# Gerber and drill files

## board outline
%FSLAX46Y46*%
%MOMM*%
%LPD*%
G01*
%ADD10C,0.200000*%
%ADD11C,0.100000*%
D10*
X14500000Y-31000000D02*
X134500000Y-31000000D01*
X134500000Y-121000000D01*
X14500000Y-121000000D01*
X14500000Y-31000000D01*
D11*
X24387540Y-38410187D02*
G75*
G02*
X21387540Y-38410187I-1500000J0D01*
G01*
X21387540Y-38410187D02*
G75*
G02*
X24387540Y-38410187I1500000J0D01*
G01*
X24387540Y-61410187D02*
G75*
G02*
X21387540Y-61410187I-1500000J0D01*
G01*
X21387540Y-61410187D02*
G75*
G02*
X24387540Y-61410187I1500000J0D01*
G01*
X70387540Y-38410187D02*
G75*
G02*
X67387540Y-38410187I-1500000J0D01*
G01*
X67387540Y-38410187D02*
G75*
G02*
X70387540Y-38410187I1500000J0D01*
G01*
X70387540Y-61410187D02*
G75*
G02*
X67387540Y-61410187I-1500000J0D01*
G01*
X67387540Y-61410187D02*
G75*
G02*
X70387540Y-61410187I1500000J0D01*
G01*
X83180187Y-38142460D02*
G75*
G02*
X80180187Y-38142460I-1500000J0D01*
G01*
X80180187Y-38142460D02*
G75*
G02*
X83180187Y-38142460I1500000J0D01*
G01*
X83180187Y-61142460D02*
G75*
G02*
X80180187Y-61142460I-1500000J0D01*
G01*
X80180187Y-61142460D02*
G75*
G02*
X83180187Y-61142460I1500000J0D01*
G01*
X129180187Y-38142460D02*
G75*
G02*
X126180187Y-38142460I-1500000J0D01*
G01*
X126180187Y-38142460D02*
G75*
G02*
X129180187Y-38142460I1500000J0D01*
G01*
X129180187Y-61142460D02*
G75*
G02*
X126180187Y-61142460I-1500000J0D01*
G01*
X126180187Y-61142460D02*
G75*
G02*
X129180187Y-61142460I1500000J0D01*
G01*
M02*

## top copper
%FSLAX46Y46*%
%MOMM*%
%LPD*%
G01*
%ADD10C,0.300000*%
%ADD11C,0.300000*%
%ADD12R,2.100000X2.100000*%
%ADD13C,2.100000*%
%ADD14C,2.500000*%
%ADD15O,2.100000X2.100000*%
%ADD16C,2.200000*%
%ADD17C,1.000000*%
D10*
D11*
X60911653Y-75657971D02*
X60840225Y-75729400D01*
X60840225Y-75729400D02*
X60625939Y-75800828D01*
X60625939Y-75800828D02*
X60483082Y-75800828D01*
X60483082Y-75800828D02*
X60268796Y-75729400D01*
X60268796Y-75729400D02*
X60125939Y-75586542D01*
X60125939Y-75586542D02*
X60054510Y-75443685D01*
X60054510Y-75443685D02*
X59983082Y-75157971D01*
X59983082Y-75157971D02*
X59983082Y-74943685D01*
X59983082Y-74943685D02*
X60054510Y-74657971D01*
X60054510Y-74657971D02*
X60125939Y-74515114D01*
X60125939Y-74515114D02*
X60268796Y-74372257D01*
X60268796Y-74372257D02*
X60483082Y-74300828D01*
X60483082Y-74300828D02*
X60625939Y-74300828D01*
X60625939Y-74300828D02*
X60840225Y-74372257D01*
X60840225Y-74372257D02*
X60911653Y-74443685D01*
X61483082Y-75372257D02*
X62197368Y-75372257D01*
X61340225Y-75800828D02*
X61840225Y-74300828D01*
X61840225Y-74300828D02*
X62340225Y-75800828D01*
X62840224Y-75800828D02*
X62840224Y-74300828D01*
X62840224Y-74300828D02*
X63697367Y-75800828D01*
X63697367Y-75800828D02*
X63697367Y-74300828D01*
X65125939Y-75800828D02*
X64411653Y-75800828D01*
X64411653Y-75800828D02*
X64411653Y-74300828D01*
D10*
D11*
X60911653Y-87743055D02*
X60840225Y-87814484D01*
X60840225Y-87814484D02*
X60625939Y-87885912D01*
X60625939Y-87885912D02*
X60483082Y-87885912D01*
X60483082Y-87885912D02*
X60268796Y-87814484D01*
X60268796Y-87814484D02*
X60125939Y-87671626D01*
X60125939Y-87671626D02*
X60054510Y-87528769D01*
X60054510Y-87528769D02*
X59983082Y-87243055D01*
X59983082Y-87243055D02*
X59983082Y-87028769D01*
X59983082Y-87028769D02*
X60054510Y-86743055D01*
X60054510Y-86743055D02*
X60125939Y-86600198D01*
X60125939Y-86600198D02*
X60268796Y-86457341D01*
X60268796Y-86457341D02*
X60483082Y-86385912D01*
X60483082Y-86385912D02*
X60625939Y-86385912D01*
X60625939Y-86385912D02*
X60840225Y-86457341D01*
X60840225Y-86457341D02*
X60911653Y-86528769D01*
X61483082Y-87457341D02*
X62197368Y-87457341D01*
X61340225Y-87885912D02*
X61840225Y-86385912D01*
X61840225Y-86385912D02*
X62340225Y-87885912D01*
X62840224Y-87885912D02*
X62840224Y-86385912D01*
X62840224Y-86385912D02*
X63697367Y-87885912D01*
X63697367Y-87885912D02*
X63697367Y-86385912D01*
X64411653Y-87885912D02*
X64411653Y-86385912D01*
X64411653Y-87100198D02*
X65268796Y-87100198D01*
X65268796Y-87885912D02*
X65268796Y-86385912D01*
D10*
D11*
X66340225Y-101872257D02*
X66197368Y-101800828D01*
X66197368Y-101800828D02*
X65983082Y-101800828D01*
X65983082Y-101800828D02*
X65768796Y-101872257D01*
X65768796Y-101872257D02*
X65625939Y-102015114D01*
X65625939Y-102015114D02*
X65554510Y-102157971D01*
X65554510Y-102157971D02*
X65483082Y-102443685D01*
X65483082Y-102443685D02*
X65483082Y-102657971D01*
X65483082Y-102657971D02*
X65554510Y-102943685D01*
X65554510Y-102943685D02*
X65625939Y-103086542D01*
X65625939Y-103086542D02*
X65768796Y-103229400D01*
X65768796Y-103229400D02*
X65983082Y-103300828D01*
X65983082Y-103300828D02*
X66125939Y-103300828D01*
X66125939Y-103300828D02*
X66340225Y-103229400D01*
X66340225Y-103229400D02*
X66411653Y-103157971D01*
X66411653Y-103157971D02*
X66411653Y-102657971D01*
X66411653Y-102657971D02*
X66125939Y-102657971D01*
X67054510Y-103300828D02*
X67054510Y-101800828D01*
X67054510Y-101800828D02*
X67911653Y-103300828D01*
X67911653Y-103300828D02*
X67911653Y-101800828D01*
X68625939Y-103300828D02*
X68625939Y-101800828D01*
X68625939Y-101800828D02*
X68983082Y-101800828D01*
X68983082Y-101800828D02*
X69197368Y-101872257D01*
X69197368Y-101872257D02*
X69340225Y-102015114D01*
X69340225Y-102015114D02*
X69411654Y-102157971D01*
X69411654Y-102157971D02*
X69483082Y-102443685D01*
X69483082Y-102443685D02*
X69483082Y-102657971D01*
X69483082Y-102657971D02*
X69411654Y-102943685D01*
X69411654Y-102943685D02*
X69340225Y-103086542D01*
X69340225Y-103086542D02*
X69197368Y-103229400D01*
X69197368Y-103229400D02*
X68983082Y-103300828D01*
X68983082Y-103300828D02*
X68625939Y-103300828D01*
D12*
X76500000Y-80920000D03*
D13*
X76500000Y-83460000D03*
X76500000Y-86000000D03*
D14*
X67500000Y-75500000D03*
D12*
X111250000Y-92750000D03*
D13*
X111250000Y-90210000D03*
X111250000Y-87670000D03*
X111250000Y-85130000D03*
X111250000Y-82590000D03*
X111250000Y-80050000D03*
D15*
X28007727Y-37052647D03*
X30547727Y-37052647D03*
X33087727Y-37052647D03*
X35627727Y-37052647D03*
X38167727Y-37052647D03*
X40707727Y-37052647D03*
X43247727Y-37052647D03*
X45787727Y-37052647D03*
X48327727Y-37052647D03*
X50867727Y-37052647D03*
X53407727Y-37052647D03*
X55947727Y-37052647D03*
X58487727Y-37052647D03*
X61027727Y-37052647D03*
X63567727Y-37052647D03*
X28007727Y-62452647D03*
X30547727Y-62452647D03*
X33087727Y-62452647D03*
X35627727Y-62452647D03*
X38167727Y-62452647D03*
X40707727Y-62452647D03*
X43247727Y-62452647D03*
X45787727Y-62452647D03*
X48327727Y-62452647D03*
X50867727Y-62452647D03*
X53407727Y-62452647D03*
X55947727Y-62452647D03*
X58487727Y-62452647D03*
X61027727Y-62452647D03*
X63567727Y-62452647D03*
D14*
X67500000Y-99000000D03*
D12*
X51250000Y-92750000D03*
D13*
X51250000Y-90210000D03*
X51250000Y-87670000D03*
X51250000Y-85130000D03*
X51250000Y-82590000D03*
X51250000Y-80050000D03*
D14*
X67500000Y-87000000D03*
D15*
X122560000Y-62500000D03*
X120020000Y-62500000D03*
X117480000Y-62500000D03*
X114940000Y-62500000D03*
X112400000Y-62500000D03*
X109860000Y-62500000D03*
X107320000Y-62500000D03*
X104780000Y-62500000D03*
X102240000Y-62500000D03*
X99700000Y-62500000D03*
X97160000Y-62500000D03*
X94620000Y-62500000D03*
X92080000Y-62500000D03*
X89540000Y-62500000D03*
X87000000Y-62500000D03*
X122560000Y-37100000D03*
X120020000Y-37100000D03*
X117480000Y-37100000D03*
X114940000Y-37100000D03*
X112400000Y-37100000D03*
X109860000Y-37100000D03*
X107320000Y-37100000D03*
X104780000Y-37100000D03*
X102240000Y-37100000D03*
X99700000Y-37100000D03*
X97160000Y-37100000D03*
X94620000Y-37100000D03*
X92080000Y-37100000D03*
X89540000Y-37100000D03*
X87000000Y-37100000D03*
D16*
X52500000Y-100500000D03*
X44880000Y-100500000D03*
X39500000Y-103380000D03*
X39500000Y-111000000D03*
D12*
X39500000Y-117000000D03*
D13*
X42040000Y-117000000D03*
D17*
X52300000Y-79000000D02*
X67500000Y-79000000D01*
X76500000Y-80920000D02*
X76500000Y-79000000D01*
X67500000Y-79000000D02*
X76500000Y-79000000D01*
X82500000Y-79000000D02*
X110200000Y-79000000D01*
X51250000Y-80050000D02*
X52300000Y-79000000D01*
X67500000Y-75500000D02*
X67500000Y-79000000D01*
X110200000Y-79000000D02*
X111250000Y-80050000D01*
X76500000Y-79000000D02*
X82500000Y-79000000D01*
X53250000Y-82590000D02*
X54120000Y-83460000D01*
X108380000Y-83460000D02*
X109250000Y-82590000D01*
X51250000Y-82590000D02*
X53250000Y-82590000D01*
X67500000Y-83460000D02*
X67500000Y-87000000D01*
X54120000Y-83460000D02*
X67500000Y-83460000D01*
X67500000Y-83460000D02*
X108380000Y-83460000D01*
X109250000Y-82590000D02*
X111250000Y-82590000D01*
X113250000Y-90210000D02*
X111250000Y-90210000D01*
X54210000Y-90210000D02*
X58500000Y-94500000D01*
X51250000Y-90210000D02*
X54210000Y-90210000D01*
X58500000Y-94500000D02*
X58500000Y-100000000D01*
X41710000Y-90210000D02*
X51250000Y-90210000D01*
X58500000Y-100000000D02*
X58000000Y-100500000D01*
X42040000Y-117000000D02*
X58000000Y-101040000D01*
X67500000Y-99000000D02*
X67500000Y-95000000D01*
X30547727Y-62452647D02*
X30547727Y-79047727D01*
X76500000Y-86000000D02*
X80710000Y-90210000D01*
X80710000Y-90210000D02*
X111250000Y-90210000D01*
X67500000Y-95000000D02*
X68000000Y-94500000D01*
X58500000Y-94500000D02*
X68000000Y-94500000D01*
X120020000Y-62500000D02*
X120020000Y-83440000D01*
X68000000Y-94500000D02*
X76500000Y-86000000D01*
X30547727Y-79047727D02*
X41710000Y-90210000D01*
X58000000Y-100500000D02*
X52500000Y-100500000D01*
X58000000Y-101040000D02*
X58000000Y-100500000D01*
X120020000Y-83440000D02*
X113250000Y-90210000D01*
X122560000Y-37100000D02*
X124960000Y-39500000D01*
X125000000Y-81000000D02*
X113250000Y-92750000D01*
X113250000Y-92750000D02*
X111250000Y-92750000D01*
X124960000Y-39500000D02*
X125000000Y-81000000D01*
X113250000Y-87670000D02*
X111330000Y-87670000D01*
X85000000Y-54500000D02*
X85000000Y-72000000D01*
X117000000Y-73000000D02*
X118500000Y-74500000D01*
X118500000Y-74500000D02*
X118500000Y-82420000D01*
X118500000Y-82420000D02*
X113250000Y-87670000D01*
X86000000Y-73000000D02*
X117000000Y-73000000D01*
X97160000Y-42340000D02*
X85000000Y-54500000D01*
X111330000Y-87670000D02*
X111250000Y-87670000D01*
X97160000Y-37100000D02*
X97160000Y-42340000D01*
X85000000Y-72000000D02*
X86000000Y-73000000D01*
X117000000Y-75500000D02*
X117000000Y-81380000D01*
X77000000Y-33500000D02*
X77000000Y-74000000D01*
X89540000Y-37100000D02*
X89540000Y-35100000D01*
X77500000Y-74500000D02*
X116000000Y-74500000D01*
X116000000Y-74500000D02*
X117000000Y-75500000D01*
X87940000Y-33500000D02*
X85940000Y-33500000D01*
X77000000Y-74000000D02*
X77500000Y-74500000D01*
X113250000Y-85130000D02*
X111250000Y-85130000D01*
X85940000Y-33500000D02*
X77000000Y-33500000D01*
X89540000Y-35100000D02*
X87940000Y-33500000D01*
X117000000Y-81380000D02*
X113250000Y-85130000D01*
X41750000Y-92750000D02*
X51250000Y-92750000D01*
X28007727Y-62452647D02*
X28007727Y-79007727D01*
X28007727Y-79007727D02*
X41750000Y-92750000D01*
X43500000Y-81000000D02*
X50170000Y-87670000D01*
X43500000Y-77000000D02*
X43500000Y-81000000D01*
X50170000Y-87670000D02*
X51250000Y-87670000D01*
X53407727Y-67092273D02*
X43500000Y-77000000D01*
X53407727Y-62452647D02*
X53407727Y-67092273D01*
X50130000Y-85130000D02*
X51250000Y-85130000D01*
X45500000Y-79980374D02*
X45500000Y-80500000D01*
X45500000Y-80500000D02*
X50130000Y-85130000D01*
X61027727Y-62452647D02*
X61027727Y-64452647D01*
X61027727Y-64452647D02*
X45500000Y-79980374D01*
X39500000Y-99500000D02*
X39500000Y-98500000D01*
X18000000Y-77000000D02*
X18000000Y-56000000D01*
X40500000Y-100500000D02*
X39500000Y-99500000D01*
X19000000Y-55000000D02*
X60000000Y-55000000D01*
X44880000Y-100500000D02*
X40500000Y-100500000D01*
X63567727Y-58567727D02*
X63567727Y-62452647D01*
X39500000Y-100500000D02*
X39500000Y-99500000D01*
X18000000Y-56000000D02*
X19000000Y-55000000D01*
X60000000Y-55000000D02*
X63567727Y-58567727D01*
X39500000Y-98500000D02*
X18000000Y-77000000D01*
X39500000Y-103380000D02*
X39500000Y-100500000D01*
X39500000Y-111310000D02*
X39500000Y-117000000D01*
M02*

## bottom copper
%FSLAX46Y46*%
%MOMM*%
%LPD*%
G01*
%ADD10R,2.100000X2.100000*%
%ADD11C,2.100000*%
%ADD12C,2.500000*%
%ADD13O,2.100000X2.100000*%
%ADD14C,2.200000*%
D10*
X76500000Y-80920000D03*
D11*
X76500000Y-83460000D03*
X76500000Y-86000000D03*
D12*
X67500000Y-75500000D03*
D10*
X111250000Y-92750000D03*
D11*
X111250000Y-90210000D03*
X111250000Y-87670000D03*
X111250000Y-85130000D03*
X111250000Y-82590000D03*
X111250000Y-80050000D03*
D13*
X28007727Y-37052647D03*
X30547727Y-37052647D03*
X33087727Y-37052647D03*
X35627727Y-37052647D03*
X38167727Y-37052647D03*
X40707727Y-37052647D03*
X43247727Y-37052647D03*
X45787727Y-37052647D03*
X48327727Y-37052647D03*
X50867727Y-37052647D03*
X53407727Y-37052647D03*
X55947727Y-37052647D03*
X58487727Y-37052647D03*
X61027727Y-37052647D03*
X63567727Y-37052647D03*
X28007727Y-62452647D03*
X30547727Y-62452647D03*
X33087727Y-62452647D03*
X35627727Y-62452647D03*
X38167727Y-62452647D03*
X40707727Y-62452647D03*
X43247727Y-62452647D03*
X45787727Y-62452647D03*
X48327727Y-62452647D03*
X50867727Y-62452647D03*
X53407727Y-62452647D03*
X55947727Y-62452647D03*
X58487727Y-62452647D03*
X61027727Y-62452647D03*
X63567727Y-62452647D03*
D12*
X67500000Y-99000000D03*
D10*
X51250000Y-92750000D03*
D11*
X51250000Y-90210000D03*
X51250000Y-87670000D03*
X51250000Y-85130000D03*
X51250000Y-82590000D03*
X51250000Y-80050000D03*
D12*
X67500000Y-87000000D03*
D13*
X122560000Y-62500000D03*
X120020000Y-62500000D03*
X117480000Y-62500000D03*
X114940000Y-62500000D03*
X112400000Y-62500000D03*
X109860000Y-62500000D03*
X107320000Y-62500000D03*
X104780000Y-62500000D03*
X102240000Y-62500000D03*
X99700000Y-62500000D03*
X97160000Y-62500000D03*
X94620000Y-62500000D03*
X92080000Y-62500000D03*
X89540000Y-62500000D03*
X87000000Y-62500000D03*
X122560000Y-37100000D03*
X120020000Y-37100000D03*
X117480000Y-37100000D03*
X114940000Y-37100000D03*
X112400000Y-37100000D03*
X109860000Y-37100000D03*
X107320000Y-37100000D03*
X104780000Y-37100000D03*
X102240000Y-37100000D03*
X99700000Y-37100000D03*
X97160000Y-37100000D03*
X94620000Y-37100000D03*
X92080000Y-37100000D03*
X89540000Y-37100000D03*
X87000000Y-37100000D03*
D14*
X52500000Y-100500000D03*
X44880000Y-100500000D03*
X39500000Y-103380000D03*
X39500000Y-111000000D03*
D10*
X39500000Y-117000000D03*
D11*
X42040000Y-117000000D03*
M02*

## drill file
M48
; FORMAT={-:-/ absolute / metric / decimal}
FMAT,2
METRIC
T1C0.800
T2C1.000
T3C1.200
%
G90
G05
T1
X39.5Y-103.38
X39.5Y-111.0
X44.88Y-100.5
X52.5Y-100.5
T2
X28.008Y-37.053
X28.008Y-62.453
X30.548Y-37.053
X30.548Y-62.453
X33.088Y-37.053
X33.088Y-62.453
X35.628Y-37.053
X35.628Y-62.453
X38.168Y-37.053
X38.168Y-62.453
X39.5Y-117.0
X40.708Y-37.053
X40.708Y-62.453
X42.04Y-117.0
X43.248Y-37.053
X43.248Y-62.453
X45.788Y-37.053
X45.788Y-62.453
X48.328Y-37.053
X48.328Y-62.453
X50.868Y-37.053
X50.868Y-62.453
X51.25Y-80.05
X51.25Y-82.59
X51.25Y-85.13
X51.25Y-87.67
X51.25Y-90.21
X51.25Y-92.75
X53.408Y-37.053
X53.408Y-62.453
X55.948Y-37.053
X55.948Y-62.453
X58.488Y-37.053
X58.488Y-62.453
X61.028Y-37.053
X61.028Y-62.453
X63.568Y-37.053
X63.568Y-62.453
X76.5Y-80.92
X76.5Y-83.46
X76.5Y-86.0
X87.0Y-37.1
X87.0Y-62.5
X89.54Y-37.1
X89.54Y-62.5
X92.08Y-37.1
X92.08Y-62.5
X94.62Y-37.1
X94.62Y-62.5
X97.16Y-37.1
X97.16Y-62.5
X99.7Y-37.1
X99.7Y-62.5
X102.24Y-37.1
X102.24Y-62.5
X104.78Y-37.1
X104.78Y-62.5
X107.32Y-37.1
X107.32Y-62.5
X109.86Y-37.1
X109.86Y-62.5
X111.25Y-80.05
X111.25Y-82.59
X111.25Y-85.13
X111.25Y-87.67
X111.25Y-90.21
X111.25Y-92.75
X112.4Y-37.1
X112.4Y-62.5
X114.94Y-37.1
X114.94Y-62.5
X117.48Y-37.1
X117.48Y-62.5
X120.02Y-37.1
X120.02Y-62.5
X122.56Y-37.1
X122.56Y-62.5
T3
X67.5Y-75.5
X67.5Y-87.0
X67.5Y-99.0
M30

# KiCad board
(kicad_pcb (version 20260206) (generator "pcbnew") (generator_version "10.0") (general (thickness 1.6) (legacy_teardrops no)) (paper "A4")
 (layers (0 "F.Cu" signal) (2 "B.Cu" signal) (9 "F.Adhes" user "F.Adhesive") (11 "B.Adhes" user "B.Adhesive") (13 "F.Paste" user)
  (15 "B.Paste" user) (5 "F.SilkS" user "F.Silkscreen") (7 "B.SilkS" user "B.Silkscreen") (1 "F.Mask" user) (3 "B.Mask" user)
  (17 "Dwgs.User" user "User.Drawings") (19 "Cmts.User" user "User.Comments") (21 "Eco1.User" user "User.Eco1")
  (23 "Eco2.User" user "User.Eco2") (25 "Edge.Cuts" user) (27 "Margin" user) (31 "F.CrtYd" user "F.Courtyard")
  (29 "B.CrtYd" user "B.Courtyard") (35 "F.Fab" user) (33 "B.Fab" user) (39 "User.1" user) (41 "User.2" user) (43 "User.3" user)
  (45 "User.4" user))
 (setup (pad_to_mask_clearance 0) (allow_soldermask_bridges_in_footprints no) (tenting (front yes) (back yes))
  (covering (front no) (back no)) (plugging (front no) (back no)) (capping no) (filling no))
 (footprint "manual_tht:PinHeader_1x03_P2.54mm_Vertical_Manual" (layer "F.Cu") (at 76.5 80.92)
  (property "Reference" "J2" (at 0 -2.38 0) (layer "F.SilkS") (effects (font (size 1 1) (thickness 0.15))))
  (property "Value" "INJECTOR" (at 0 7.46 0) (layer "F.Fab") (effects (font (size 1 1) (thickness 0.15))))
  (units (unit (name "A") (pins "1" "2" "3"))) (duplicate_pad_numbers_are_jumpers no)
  (pad "1" thru_hole rect (at 0 0) (size 2.1 2.1) (drill 1) (layers "*.Cu" "*.Mask") (remove_unused_layers no) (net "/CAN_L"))
  (pad "2" thru_hole circle (at 0 2.54) (size 2.1 2.1) (drill 1) (layers "*.Cu" "*.Mask") (remove_unused_layers no) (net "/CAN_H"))
  (pad "3" thru_hole circle (at 0 5.08) (size 2.1 2.1) (drill 1) (layers "*.Cu" "*.Mask") (remove_unused_layers no) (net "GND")))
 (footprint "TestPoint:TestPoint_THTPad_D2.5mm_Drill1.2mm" (layer "F.Cu") (at 67.5 75.5)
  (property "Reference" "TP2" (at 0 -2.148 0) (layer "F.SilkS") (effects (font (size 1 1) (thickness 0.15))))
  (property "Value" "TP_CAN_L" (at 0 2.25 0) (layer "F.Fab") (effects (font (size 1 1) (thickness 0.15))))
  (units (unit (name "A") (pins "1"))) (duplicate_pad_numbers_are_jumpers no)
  (pad "1" thru_hole circle (at 0 0) (size 2.5 2.5) (drill 1.2) (layers "*.Cu" "*.Mask") (remove_unused_layers no) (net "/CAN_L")))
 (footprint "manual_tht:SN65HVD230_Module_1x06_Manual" (layer "F.Cu") (at 111.25 92.75 180)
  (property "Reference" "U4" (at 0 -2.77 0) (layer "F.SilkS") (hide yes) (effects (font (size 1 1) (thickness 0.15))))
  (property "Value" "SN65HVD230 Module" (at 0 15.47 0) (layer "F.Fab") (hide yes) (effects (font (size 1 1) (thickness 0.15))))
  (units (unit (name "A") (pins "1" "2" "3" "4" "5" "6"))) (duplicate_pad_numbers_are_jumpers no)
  (pad "1" thru_hole rect (at 0 0 180) (size 2.1 2.1) (drill 1) (layers "*.Cu" "*.Mask") (remove_unused_layers no) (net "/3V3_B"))
  (pad "2" thru_hole circle (at 0 2.54 180) (size 2.1 2.1) (drill 1) (layers "*.Cu" "*.Mask") (remove_unused_layers no) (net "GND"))
  (pad "3" thru_hole circle (at 0 5.08 180) (size 2.1 2.1) (drill 1) (layers "*.Cu" "*.Mask") (remove_unused_layers no) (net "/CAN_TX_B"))
  (pad "4" thru_hole circle (at 0 7.62 180) (size 2.1 2.1) (drill 1) (layers "*.Cu" "*.Mask") (remove_unused_layers no) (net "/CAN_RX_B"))
  (pad "5" thru_hole circle (at 0 10.16 180) (size 2.1 2.1) (drill 1) (layers "*.Cu" "*.Mask") (remove_unused_layers no) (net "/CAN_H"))
  (pad "6" thru_hole circle (at 0 12.7 180) (size 2.1 2.1) (drill 1) (layers "*.Cu" "*.Mask") (remove_unused_layers no) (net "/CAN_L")))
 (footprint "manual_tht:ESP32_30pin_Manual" (layer "F.Cu") (at 45.02754 48.980187 -90)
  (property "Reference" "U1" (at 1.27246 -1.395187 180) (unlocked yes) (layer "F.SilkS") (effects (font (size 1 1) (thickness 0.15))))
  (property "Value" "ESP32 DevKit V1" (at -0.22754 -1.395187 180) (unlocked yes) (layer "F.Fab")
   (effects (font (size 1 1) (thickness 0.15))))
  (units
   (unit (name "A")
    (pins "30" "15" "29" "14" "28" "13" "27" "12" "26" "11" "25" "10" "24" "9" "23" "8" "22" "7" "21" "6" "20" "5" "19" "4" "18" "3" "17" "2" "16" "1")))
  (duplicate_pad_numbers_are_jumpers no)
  (fp_circle (center -10.57 22.14) (end -10.57 23.64) (stroke (width 0.1) (type default)) (fill no) (layer "Edge.Cuts"))
  (fp_circle (center 12.43 22.14) (end 12.43 23.64) (stroke (width 0.1) (type default)) (fill no) (layer "Edge.Cuts"))
  (fp_circle (center -10.57 -23.86) (end -10.57 -22.36) (stroke (width 0.1) (type default)) (fill no) (layer "Edge.Cuts"))
  (fp_circle (center 12.43 -23.86) (end 12.43 -22.36) (stroke (width 0.1) (type default)) (fill no) (layer "Edge.Cuts"))
  (pad "1" thru_hole oval (at -11.92754 17.019813 180) (size 2.1 2.1) (drill 1) (layers "*.Cu" "*.Mask") (remove_unused_layers no)
   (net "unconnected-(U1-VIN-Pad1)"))
  (pad "2" thru_hole oval (at -11.92754 14.479813 180) (size 2.1 2.1) (drill 1) (layers "*.Cu" "*.Mask") (remove_unused_layers no)
   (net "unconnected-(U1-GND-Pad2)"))
  (pad "3" thru_hole oval (at -11.92754 11.939813 180) (size 2.1 2.1) (drill 1) (layers "*.Cu" "*.Mask") (remove_unused_layers no)
   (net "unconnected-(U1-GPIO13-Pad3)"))
  (pad "4" thru_hole oval (at -11.92754 9.399813 180) (size 2.1 2.1) (drill 1) (layers "*.Cu" "*.Mask") (remove_unused_layers no)
   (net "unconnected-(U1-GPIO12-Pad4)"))
  (pad "5" thru_hole oval (at -11.92754 6.859813 180) (size 2.1 2.1) (drill 1) (layers "*.Cu" "*.Mask") (remove_unused_layers no)
   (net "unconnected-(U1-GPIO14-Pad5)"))
  (pad "6" thru_hole oval (at -11.92754 4.319813 180) (size 2.1 2.1) (drill 1) (layers "*.Cu" "*.Mask") (remove_unused_layers no)
   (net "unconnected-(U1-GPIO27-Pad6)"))
  (pad "7" thru_hole oval (at -11.92754 1.779813 180) (size 2.1 2.1) (drill 1) (layers "*.Cu" "*.Mask") (remove_unused_layers no)
   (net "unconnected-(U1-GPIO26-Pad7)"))
  (pad "8" thru_hole oval (at -11.92754 -0.760187 180) (size 2.1 2.1) (drill 1) (layers "*.Cu" "*.Mask") (remove_unused_layers no)
   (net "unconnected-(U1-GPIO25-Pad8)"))
  (pad "9" thru_hole oval (at -11.92754 -3.300187 180) (size 2.1 2.1) (drill 1) (layers "*.Cu" "*.Mask") (remove_unused_layers no)
   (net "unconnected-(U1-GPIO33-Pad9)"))
  (pad "10" thru_hole oval (at -11.92754 -5.840187 180) (size 2.1 2.1) (drill 1) (layers "*.Cu" "*.Mask") (remove_unused_layers no)
   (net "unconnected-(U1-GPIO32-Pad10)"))
  (pad "11" thru_hole oval (at -11.92754 -8.380187 180) (size 2.1 2.1) (drill 1) (layers "*.Cu" "*.Mask") (remove_unused_layers no)
   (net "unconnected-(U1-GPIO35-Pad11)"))
  (pad "12" thru_hole oval (at -11.92754 -10.920187 180) (size 2.1 2.1) (drill 1) (layers "*.Cu" "*.Mask") (remove_unused_layers no)
   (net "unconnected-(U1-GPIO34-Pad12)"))
  (pad "13" thru_hole oval (at -11.92754 -13.460187 180) (size 2.1 2.1) (drill 1) (layers "*.Cu" "*.Mask") (remove_unused_layers no)
   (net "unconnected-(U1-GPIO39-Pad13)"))
  (pad "14" thru_hole oval (at -11.92754 -16.000187 180) (size 2.1 2.1) (drill 1) (layers "*.Cu" "*.Mask") (remove_unused_layers no)
   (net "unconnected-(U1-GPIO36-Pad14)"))
  (pad "15" thru_hole oval (at -11.92754 -18.540187 180) (size 2.1 2.1) (drill 1) (layers "*.Cu" "*.Mask") (remove_unused_layers no)
   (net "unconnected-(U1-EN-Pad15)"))
  (pad "16" thru_hole oval (at 13.47246 17.019813 180) (size 2.1 2.1) (drill 1) (layers "*.Cu" "*.Mask") (remove_unused_layers no)
   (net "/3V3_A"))
  (pad "17" thru_hole oval (at 13.47246 14.479813 180) (size 2.1 2.1) (drill 1) (layers "*.Cu" "*.Mask") (remove_unused_layers no)
   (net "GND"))
  (pad "18" thru_hole oval (at 13.47246 11.939813 180) (size 2.1 2.1) (drill 1) (layers "*.Cu" "*.Mask") (remove_unused_layers no)
   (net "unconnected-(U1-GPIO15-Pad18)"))
  (pad "19" thru_hole oval (at 13.47246 9.399813 180) (size 2.1 2.1) (drill 1) (layers "*.Cu" "*.Mask") (remove_unused_layers no)
   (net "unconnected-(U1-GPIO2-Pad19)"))
  (pad "20" thru_hole oval (at 13.47246 6.859813 180) (size 2.1 2.1) (drill 1) (layers "*.Cu" "*.Mask" "Dwgs.User")
   (remove_unused_layers no) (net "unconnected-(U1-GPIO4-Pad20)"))
  (pad "21" thru_hole oval (at 13.47246 4.319813 180) (size 2.1 2.1) (drill 1) (layers "*.Cu" "*.Mask") (remove_unused_layers no)
   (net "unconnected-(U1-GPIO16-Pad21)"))
  (pad "22" thru_hole oval (at 13.47246 1.779813 180) (size 2.1 2.1) (drill 1) (layers "*.Cu" "*.Mask") (remove_unused_layers no)
   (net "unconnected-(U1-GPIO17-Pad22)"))
  (pad "23" thru_hole oval (at 13.47246 -0.760187 180) (size 2.1 2.1) (drill 1) (layers "*.Cu" "*.Mask") (remove_unused_layers no)
   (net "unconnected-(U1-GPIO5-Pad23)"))
  (pad "24" thru_hole oval (at 13.47246 -3.300187 180) (size 2.1 2.1) (drill 1) (layers "*.Cu" "*.Mask") (remove_unused_layers no)
   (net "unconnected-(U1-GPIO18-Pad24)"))
  (pad "25" thru_hole oval (at 13.47246 -5.840187 180) (size 2.1 2.1) (drill 1) (layers "*.Cu" "*.Mask") (remove_unused_layers no)
   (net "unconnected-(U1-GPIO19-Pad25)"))
  (pad "26" thru_hole oval (at 13.47246 -8.380187 180) (size 2.1 2.1) (drill 1) (layers "*.Cu" "*.Mask") (remove_unused_layers no)
   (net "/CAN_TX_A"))
  (pad "27" thru_hole oval (at 13.47246 -10.920187 180) (size 2.1 2.1) (drill 1) (layers "*.Cu" "*.Mask") (remove_unused_layers no)
   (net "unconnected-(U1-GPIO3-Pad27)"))
  (pad "28" thru_hole oval (at 13.47246 -13.460187 180) (size 2.1 2.1) (drill 1) (layers "*.Cu" "*.Mask") (remove_unused_layers no)
   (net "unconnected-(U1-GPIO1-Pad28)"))
  (pad "29" thru_hole oval (at 13.47246 -16.000187 180) (size 2.1 2.1) (drill 1) (layers "*.Cu" "*.Mask") (remove_unused_layers no)
   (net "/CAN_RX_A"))
  (pad "30" thru_hole oval (at 13.47246 -18.540187 180) (size 2.1 2.1) (drill 1) (layers "*.Cu" "*.Mask") (remove_unused_layers no)
   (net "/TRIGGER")))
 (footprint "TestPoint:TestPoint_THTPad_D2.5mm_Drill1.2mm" (layer "F.Cu") (at 67.5 99)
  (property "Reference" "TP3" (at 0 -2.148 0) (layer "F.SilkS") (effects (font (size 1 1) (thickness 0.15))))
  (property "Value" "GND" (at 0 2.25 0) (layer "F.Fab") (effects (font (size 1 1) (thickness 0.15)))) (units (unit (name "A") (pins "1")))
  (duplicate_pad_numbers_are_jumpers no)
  (pad "1" thru_hole circle (at 0 0) (size 2.5 2.5) (drill 1.2) (layers "*.Cu" "*.Mask") (remove_unused_layers no) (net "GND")))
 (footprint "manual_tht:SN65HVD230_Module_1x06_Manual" (layer "F.Cu") (at 51.25 92.75 180)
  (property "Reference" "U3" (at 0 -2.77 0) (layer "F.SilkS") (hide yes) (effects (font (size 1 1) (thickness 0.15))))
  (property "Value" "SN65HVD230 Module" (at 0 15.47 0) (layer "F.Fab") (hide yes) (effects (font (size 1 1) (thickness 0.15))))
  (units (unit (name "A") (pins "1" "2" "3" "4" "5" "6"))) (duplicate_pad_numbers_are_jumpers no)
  (pad "1" thru_hole rect (at 0 0 180) (size 2.1 2.1) (drill 1) (layers "*.Cu" "*.Mask") (remove_unused_layers no) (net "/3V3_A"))
  (pad "2" thru_hole circle (at 0 2.54 180) (size 2.1 2.1) (drill 1) (layers "*.Cu" "*.Mask") (remove_unused_layers no) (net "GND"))
  (pad "3" thru_hole circle (at 0 5.08 180) (size 2.1 2.1) (drill 1) (layers "*.Cu" "*.Mask") (remove_unused_layers no) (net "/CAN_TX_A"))
  (pad "4" thru_hole circle (at 0 7.62 180) (size 2.1 2.1) (drill 1) (layers "*.Cu" "*.Mask") (remove_unused_layers no) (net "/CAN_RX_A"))
  (pad "5" thru_hole circle (at 0 10.16 180) (size 2.1 2.1) (drill 1) (layers "*.Cu" "*.Mask") (remove_unused_layers no) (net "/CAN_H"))
  (pad "6" thru_hole circle (at 0 12.7 180) (size 2.1 2.1) (drill 1) (layers "*.Cu" "*.Mask") (remove_unused_layers no) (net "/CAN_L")))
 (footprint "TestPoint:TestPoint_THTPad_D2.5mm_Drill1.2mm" (layer "F.Cu") (at 67.5 87)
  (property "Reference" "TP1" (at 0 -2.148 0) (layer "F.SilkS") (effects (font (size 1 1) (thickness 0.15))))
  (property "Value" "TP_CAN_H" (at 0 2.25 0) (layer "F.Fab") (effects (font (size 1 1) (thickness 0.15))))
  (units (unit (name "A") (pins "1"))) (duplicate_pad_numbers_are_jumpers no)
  (pad "1" thru_hole circle (at 0 0) (size 2.5 2.5) (drill 1.2) (layers "*.Cu" "*.Mask") (remove_unused_layers no) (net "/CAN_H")))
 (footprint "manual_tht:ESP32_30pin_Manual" (layer "F.Cu") (at 105.540187 50.57246 90)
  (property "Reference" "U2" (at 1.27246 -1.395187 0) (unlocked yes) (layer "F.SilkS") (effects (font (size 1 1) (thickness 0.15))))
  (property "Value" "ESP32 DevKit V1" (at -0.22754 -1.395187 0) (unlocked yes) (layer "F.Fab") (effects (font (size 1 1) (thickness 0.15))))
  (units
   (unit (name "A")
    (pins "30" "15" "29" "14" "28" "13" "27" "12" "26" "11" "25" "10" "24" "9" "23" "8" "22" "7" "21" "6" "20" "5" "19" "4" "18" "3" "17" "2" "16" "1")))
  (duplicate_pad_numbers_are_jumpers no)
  (fp_circle (center 12.43 -23.86) (end 12.43 -22.36) (stroke (width 0.1) (type default)) (fill no) (layer "Edge.Cuts"))
  (fp_circle (center -10.57 -23.86) (end -10.57 -22.36) (stroke (width 0.1) (type default)) (fill no) (layer "Edge.Cuts"))
  (fp_circle (center 12.43 22.14) (end 12.43 23.64) (stroke (width 0.1) (type default)) (fill no) (layer "Edge.Cuts"))
  (fp_circle (center -10.57 22.14) (end -10.57 23.64) (stroke (width 0.1) (type default)) (fill no) (layer "Edge.Cuts"))
  (pad "1" thru_hole oval (at -11.92754 17.019813) (size 2.1 2.1) (drill 1) (layers "*.Cu" "*.Mask") (remove_unused_layers no)
   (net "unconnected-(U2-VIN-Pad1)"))
  (pad "2" thru_hole oval (at -11.92754 14.479813) (size 2.1 2.1) (drill 1) (layers "*.Cu" "*.Mask") (remove_unused_layers no) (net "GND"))
  (pad "3" thru_hole oval (at -11.92754 11.939813) (size 2.1 2.1) (drill 1) (layers "*.Cu" "*.Mask") (remove_unused_layers no)
   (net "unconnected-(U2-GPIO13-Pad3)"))
  (pad "4" thru_hole oval (at -11.92754 9.399813) (size 2.1 2.1) (drill 1) (layers "*.Cu" "*.Mask") (remove_unused_layers no)
   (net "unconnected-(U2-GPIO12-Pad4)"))
  (pad "5" thru_hole oval (at -11.92754 6.859813) (size 2.1 2.1) (drill 1) (layers "*.Cu" "*.Mask") (remove_unused_layers no)
   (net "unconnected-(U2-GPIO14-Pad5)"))
  (pad "6" thru_hole oval (at -11.92754 4.319813) (size 2.1 2.1) (drill 1) (layers "*.Cu" "*.Mask") (remove_unused_layers no)
   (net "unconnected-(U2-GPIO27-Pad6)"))
  (pad "7" thru_hole oval (at -11.92754 1.779813) (size 2.1 2.1) (drill 1) (layers "*.Cu" "*.Mask") (remove_unused_layers no)
   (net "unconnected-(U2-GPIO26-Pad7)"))
  (pad "8" thru_hole oval (at -11.92754 -0.760187) (size 2.1 2.1) (drill 1) (layers "*.Cu" "*.Mask") (remove_unused_layers no)
   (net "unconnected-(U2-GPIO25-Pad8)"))
  (pad "9" thru_hole oval (at -11.92754 -3.300187) (size 2.1 2.1) (drill 1) (layers "*.Cu" "*.Mask") (remove_unused_layers no)
   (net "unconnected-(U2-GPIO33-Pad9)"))
  (pad "10" thru_hole oval (at -11.92754 -5.840187) (size 2.1 2.1) (drill 1) (layers "*.Cu" "*.Mask") (remove_unused_layers no)
   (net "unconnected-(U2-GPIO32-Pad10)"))
  (pad "11" thru_hole oval (at -11.92754 -8.380187) (size 2.1 2.1) (drill 1) (layers "*.Cu" "*.Mask") (remove_unused_layers no)
   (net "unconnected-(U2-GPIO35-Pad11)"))
  (pad "12" thru_hole oval (at -11.92754 -10.920187) (size 2.1 2.1) (drill 1) (layers "*.Cu" "*.Mask") (remove_unused_layers no)
   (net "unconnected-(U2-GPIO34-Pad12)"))
  (pad "13" thru_hole oval (at -11.92754 -13.460187) (size 2.1 2.1) (drill 1) (layers "*.Cu" "*.Mask") (remove_unused_layers no)
   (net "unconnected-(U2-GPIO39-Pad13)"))
  (pad "14" thru_hole oval (at -11.92754 -16.000187) (size 2.1 2.1) (drill 1) (layers "*.Cu" "*.Mask") (remove_unused_layers no)
   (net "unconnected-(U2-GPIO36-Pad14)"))
  (pad "15" thru_hole oval (at -11.92754 -18.540187) (size 2.1 2.1) (drill 1) (layers "*.Cu" "*.Mask") (remove_unused_layers no)
   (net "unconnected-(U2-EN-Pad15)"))
  (pad "16" thru_hole oval (at 13.47246 17.019813) (size 2.1 2.1) (drill 1) (layers "*.Cu" "*.Mask") (remove_unused_layers no)
   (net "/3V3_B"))
  (pad "17" thru_hole oval (at 13.47246 14.479813) (size 2.1 2.1) (drill 1) (layers "*.Cu" "*.Mask") (remove_unused_layers no)
   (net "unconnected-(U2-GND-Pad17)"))
  (pad "18" thru_hole oval (at 13.47246 11.939813) (size 2.1 2.1) (drill 1) (layers "*.Cu" "*.Mask") (remove_unused_layers no)
   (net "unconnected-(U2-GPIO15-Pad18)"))
  (pad "19" thru_hole oval (at 13.47246 9.399813) (size 2.1 2.1) (drill 1) (layers "*.Cu" "*.Mask") (remove_unused_layers no)
   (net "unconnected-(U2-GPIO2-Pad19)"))
  (pad "20" thru_hole oval (at 13.47246 6.859813) (size 2.1 2.1) (drill 1) (layers "*.Cu" "*.Mask" "Dwgs.User") (remove_unused_layers no)
   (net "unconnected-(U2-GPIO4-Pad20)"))
  (pad "21" thru_hole oval (at 13.47246 4.319813) (size 2.1 2.1) (drill 1) (layers "*.Cu" "*.Mask") (remove_unused_layers no)
   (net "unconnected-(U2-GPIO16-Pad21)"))
  (pad "22" thru_hole oval (at 13.47246 1.779813) (size 2.1 2.1) (drill 1) (layers "*.Cu" "*.Mask") (remove_unused_layers no)
   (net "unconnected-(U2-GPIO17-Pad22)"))
  (pad "23" thru_hole oval (at 13.47246 -0.760187) (size 2.1 2.1) (drill 1) (layers "*.Cu" "*.Mask") (remove_unused_layers no)
   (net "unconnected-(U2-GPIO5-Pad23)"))
  (pad "24" thru_hole oval (at 13.47246 -3.300187) (size 2.1 2.1) (drill 1) (layers "*.Cu" "*.Mask") (remove_unused_layers no)
   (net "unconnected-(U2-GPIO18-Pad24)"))
  (pad "25" thru_hole oval (at 13.47246 -5.840187) (size 2.1 2.1) (drill 1) (layers "*.Cu" "*.Mask") (remove_unused_layers no)
   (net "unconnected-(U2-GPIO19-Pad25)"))
  (pad "26" thru_hole oval (at 13.47246 -8.380187) (size 2.1 2.1) (drill 1) (layers "*.Cu" "*.Mask") (remove_unused_layers no)
   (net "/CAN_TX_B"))
  (pad "27" thru_hole oval (at 13.47246 -10.920187) (size 2.1 2.1) (drill 1) (layers "*.Cu" "*.Mask") (remove_unused_layers no)
   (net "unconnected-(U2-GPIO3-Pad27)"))
  (pad "28" thru_hole oval (at 13.47246 -13.460187) (size 2.1 2.1) (drill 1) (layers "*.Cu" "*.Mask") (remove_unused_layers no)
   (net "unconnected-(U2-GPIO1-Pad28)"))
  (pad "29" thru_hole oval (at 13.47246 -16.000187) (size 2.1 2.1) (drill 1) (layers "*.Cu" "*.Mask") (remove_unused_layers no)
   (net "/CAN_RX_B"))
  (pad "30" thru_hole oval (at 13.47246 -18.540187) (size 2.1 2.1) (drill 1) (layers "*.Cu" "*.Mask") (remove_unused_layers no)
   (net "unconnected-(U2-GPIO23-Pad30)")))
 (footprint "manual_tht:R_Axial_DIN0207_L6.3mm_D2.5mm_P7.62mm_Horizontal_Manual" (layer "F.Cu") (at 52.5 100.5 180)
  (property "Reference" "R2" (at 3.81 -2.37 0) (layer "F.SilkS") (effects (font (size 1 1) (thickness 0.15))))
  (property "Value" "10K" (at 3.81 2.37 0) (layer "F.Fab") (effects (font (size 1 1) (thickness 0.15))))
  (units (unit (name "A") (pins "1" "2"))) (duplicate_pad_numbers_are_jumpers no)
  (pad "1" thru_hole circle (at 0 0 180) (size 2.2 2.2) (drill 0.8) (layers "*.Cu" "*.Mask") (remove_unused_layers no) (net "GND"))
  (pad "2" thru_hole circle (at 7.62 0 180) (size 2.2 2.2) (drill 0.8) (layers "*.Cu" "*.Mask") (remove_unused_layers no) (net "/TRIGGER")))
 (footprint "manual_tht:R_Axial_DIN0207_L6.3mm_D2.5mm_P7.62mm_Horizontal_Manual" (layer "F.Cu") (at 39.5 103.38 -90)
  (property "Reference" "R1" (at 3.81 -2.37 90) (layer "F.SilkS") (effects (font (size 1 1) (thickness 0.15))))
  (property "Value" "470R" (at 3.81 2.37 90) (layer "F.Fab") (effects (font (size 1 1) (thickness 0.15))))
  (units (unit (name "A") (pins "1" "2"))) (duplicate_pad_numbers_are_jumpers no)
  (pad "1" thru_hole circle (at 0 0 270) (size 2.2 2.2) (drill 0.8) (layers "*.Cu" "*.Mask") (remove_unused_layers no) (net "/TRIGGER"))
  (pad "2" thru_hole circle (at 7.62 0 270) (size 2.2 2.2) (drill 0.8) (layers "*.Cu" "*.Mask") (remove_unused_layers no)
   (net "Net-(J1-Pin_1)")))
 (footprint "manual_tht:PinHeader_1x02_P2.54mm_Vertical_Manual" (layer "F.Cu") (at 39.5 117 90)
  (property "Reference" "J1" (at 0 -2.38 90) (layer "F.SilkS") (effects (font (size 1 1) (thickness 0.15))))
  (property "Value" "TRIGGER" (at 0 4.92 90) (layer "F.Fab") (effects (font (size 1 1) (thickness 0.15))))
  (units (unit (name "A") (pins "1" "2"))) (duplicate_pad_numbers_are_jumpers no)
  (pad "1" thru_hole rect (at 0 0 90) (size 2.1 2.1) (drill 1) (layers "*.Cu" "*.Mask") (remove_unused_layers no) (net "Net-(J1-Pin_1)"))
  (pad "2" thru_hole circle (at 0 2.54 90) (size 2.1 2.1) (drill 1) (layers "*.Cu" "*.Mask") (remove_unused_layers no) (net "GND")))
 (gr_rect (start 14.5 31) (end 134.5 121) (stroke (width 0.2) (type default)) (fill no) (layer "Edge.Cuts"))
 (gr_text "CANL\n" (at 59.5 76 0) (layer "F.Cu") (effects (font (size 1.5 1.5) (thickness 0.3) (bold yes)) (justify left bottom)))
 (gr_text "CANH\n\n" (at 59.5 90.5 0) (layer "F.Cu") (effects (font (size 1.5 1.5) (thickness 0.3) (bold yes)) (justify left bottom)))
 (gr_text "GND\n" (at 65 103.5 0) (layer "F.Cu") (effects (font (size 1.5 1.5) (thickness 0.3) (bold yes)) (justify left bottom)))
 (segment (start 52.3 79) (end 67.5 79) (width 1) (layer "F.Cu") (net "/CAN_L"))
 (segment (start 76.5 80.92) (end 76.5 79) (width 1) (layer "F.Cu") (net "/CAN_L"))
 (segment (start 67.5 79) (end 76.5 79) (width 1) (layer "F.Cu") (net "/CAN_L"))
 (segment (start 82.5 79) (end 110.2 79) (width 1) (layer "F.Cu") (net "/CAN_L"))
 (segment (start 51.25 80.05) (end 52.3 79) (width 1) (layer "F.Cu") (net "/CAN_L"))
 (segment (start 67.5 75.5) (end 67.5 79) (width 1) (layer "F.Cu") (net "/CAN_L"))
 (segment (start 110.2 79) (end 111.25 80.05) (width 1) (layer "F.Cu") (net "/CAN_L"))
 (segment (start 76.5 79) (end 82.5 79) (width 1) (layer "F.Cu") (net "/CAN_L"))
 (segment (start 53.25 82.59) (end 54.12 83.46) (width 1) (layer "F.Cu") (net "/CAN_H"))
 (segment (start 108.38 83.46) (end 109.25 82.59) (width 1) (layer "F.Cu") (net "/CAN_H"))
 (segment (start 51.25 82.59) (end 53.25 82.59) (width 1) (layer "F.Cu") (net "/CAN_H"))
 (segment (start 67.5 83.46) (end 67.5 87) (width 1) (layer "F.Cu") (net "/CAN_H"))
 (segment (start 54.12 83.46) (end 67.5 83.46) (width 1) (layer "F.Cu") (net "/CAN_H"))
 (segment (start 67.5 83.46) (end 108.38 83.46) (width 1) (layer "F.Cu") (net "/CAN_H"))
 (segment (start 109.25 82.59) (end 111.25 82.59) (width 1) (layer "F.Cu") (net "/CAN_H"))
 (segment (start 113.25 90.21) (end 111.25 90.21) (width 1) (layer "F.Cu") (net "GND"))
 (segment (start 54.21 90.21) (end 58.5 94.5) (width 1) (layer "F.Cu") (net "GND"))
 (segment (start 51.25 90.21) (end 54.21 90.21) (width 1) (layer "F.Cu") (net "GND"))
 (segment (start 58.5 94.5) (end 58.5 100) (width 1) (layer "F.Cu") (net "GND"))
 (segment (start 41.71 90.21) (end 51.25 90.21) (width 1) (layer "F.Cu") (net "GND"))
 (segment (start 58.5 100) (end 58 100.5) (width 1) (layer "F.Cu") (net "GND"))
 (segment (start 42.04 117) (end 58 101.04) (width 1) (layer "F.Cu") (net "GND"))
 (segment (start 67.5 99) (end 67.5 95) (width 1) (layer "F.Cu") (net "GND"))
 (segment (start 30.547727 62.452647) (end 30.547727 79.047727) (width 1) (layer "F.Cu") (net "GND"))
 (segment (start 76.5 86) (end 80.71 90.21) (width 1) (layer "F.Cu") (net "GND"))
 (segment (start 80.71 90.21) (end 111.25 90.21) (width 1) (layer "F.Cu") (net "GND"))
 (segment (start 67.5 95) (end 68 94.5) (width 1) (layer "F.Cu") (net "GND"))
 (segment (start 58.5 94.5) (end 68 94.5) (width 1) (layer "F.Cu") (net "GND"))
 (segment (start 120.02 62.5) (end 120.02 83.44) (width 1) (layer "F.Cu") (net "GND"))
 (segment (start 68 94.5) (end 76.5 86) (width 1) (layer "F.Cu") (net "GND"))
 (segment (start 30.547727 79.047727) (end 41.71 90.21) (width 1) (layer "F.Cu") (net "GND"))
 (segment (start 58 100.5) (end 52.5 100.5) (width 1) (layer "F.Cu") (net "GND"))
 (segment (start 58 101.04) (end 58 100.5) (width 1) (layer "F.Cu") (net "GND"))
 (segment (start 120.02 83.44) (end 113.25 90.21) (width 1) (layer "F.Cu") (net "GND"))
 (segment (start 122.56 37.1) (end 124.96 39.5) (width 1) (layer "F.Cu") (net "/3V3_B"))
 (segment (start 125 81) (end 113.25 92.75) (width 1) (layer "F.Cu") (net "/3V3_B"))
 (segment (start 113.25 92.75) (end 111.25 92.75) (width 1) (layer "F.Cu") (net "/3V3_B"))
 (segment (start 124.96 39.5) (end 125 81) (width 1) (layer "F.Cu") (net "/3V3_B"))
 (segment (start 113.25 87.67) (end 111.33 87.67) (width 1) (layer "F.Cu") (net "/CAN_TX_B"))
 (segment (start 85 54.5) (end 85 72) (width 1) (layer "F.Cu") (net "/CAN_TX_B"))
 (segment (start 117 73) (end 118.5 74.5) (width 1) (layer "F.Cu") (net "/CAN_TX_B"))
 (segment (start 118.5 74.5) (end 118.5 82.42) (width 1) (layer "F.Cu") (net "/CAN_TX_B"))
 (segment (start 118.5 82.42) (end 113.25 87.67) (width 1) (layer "F.Cu") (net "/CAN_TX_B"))
 (segment (start 86 73) (end 117 73) (width 1) (layer "F.Cu") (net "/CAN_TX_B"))
 (segment (start 97.16 42.34) (end 85 54.5) (width 1) (layer "F.Cu") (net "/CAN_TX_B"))
 (segment (start 111.33 87.67) (end 111.25 87.67) (width 1) (layer "F.Cu") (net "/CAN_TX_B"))
 (segment (start 97.16 37.1) (end 97.16 42.34) (width 1) (layer "F.Cu") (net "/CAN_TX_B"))
 (segment (start 85 72) (end 86 73) (width 1) (layer "F.Cu") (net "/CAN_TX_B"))
 (segment (start 117 75.5) (end 117 81.38) (width 1) (layer "F.Cu") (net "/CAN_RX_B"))
 (segment (start 77 33.5) (end 77 74) (width 1) (layer "F.Cu") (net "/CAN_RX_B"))
 (segment (start 89.54 37.1) (end 89.54 35.1) (width 1) (layer "F.Cu") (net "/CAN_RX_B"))
 (segment (start 77.5 74.5) (end 116 74.5) (width 1) (layer "F.Cu") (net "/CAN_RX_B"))
 (segment (start 116 74.5) (end 117 75.5) (width 1) (layer "F.Cu") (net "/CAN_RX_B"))
 (segment (start 87.94 33.5) (end 85.94 33.5) (width 1) (layer "F.Cu") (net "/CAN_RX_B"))
 (segment (start 77 74) (end 77.5 74.5) (width 1) (layer "F.Cu") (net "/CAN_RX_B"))
 (segment (start 113.25 85.13) (end 111.25 85.13) (width 1) (layer "F.Cu") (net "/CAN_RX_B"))
 (segment (start 85.94 33.5) (end 77 33.5) (width 1) (layer "F.Cu") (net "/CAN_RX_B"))
 (segment (start 89.54 35.1) (end 87.94 33.5) (width 1) (layer "F.Cu") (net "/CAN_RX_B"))
 (segment (start 117 81.38) (end 113.25 85.13) (width 1) (layer "F.Cu") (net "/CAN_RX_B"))
 (segment (start 41.75 92.75) (end 51.25 92.75) (width 1) (layer "F.Cu") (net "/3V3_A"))
 (segment (start 28.007727 62.452647) (end 28.007727 79.007727) (width 1) (layer "F.Cu") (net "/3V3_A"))
 (segment (start 28.007727 79.007727) (end 41.75 92.75) (width 1) (layer "F.Cu") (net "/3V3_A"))
 (segment (start 43.5 81) (end 50.17 87.67) (width 1) (layer "F.Cu") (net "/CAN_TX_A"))
 (segment (start 43.5 77) (end 43.5 81) (width 1) (layer "F.Cu") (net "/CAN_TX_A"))
 (segment (start 50.17 87.67) (end 51.25 87.67) (width 1) (layer "F.Cu") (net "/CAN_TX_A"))
 (segment (start 53.407727 67.092273) (end 43.5 77) (width 1) (layer "F.Cu") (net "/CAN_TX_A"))
 (segment (start 53.407727 62.452647) (end 53.407727 67.092273) (width 1) (layer "F.Cu") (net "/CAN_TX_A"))
 (segment (start 50.13 85.13) (end 51.25 85.13) (width 1) (layer "F.Cu") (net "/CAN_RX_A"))
 (segment (start 45.5 79.980374) (end 45.5 80.5) (width 1) (layer "F.Cu") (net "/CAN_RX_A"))
 (segment (start 45.5 80.5) (end 50.13 85.13) (width 1) (layer "F.Cu") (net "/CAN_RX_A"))
 (segment (start 61.027727 62.452647) (end 61.027727 64.452647) (width 1) (layer "F.Cu") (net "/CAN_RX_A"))
 (segment (start 61.027727 64.452647) (end 45.5 79.980374) (width 1) (layer "F.Cu") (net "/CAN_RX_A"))
 (segment (start 39.5 99.5) (end 39.5 98.5) (width 1) (layer "F.Cu") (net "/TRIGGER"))
 (segment (start 18 77) (end 18 56) (width 1) (layer "F.Cu") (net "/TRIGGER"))
 (segment (start 40.5 100.5) (end 39.5 99.5) (width 1) (layer "F.Cu") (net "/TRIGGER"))
 (segment (start 19 55) (end 60 55) (width 1) (layer "F.Cu") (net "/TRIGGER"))
 (segment (start 44.88 100.5) (end 40.5 100.5) (width 1) (layer "F.Cu") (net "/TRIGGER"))
 (segment (start 63.567727 58.567727) (end 63.567727 62.452647) (width 1) (layer "F.Cu") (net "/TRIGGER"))
 (segment (start 39.5 100.5) (end 39.5 99.5) (width 1) (layer "F.Cu") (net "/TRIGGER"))
 (segment (start 18 56) (end 19 55) (width 1) (layer "F.Cu") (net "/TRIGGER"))
 (segment (start 60 55) (end 63.567727 58.567727) (width 1) (layer "F.Cu") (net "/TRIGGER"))
 (segment (start 39.5 98.5) (end 18 77) (width 1) (layer "F.Cu") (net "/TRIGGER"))
 (segment (start 39.5 103.38) (end 39.5 100.5) (width 1) (layer "F.Cu") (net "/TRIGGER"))
 (segment (start 39.5 111.31) (end 39.5 117) (width 1) (layer "F.Cu") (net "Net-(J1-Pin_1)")))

